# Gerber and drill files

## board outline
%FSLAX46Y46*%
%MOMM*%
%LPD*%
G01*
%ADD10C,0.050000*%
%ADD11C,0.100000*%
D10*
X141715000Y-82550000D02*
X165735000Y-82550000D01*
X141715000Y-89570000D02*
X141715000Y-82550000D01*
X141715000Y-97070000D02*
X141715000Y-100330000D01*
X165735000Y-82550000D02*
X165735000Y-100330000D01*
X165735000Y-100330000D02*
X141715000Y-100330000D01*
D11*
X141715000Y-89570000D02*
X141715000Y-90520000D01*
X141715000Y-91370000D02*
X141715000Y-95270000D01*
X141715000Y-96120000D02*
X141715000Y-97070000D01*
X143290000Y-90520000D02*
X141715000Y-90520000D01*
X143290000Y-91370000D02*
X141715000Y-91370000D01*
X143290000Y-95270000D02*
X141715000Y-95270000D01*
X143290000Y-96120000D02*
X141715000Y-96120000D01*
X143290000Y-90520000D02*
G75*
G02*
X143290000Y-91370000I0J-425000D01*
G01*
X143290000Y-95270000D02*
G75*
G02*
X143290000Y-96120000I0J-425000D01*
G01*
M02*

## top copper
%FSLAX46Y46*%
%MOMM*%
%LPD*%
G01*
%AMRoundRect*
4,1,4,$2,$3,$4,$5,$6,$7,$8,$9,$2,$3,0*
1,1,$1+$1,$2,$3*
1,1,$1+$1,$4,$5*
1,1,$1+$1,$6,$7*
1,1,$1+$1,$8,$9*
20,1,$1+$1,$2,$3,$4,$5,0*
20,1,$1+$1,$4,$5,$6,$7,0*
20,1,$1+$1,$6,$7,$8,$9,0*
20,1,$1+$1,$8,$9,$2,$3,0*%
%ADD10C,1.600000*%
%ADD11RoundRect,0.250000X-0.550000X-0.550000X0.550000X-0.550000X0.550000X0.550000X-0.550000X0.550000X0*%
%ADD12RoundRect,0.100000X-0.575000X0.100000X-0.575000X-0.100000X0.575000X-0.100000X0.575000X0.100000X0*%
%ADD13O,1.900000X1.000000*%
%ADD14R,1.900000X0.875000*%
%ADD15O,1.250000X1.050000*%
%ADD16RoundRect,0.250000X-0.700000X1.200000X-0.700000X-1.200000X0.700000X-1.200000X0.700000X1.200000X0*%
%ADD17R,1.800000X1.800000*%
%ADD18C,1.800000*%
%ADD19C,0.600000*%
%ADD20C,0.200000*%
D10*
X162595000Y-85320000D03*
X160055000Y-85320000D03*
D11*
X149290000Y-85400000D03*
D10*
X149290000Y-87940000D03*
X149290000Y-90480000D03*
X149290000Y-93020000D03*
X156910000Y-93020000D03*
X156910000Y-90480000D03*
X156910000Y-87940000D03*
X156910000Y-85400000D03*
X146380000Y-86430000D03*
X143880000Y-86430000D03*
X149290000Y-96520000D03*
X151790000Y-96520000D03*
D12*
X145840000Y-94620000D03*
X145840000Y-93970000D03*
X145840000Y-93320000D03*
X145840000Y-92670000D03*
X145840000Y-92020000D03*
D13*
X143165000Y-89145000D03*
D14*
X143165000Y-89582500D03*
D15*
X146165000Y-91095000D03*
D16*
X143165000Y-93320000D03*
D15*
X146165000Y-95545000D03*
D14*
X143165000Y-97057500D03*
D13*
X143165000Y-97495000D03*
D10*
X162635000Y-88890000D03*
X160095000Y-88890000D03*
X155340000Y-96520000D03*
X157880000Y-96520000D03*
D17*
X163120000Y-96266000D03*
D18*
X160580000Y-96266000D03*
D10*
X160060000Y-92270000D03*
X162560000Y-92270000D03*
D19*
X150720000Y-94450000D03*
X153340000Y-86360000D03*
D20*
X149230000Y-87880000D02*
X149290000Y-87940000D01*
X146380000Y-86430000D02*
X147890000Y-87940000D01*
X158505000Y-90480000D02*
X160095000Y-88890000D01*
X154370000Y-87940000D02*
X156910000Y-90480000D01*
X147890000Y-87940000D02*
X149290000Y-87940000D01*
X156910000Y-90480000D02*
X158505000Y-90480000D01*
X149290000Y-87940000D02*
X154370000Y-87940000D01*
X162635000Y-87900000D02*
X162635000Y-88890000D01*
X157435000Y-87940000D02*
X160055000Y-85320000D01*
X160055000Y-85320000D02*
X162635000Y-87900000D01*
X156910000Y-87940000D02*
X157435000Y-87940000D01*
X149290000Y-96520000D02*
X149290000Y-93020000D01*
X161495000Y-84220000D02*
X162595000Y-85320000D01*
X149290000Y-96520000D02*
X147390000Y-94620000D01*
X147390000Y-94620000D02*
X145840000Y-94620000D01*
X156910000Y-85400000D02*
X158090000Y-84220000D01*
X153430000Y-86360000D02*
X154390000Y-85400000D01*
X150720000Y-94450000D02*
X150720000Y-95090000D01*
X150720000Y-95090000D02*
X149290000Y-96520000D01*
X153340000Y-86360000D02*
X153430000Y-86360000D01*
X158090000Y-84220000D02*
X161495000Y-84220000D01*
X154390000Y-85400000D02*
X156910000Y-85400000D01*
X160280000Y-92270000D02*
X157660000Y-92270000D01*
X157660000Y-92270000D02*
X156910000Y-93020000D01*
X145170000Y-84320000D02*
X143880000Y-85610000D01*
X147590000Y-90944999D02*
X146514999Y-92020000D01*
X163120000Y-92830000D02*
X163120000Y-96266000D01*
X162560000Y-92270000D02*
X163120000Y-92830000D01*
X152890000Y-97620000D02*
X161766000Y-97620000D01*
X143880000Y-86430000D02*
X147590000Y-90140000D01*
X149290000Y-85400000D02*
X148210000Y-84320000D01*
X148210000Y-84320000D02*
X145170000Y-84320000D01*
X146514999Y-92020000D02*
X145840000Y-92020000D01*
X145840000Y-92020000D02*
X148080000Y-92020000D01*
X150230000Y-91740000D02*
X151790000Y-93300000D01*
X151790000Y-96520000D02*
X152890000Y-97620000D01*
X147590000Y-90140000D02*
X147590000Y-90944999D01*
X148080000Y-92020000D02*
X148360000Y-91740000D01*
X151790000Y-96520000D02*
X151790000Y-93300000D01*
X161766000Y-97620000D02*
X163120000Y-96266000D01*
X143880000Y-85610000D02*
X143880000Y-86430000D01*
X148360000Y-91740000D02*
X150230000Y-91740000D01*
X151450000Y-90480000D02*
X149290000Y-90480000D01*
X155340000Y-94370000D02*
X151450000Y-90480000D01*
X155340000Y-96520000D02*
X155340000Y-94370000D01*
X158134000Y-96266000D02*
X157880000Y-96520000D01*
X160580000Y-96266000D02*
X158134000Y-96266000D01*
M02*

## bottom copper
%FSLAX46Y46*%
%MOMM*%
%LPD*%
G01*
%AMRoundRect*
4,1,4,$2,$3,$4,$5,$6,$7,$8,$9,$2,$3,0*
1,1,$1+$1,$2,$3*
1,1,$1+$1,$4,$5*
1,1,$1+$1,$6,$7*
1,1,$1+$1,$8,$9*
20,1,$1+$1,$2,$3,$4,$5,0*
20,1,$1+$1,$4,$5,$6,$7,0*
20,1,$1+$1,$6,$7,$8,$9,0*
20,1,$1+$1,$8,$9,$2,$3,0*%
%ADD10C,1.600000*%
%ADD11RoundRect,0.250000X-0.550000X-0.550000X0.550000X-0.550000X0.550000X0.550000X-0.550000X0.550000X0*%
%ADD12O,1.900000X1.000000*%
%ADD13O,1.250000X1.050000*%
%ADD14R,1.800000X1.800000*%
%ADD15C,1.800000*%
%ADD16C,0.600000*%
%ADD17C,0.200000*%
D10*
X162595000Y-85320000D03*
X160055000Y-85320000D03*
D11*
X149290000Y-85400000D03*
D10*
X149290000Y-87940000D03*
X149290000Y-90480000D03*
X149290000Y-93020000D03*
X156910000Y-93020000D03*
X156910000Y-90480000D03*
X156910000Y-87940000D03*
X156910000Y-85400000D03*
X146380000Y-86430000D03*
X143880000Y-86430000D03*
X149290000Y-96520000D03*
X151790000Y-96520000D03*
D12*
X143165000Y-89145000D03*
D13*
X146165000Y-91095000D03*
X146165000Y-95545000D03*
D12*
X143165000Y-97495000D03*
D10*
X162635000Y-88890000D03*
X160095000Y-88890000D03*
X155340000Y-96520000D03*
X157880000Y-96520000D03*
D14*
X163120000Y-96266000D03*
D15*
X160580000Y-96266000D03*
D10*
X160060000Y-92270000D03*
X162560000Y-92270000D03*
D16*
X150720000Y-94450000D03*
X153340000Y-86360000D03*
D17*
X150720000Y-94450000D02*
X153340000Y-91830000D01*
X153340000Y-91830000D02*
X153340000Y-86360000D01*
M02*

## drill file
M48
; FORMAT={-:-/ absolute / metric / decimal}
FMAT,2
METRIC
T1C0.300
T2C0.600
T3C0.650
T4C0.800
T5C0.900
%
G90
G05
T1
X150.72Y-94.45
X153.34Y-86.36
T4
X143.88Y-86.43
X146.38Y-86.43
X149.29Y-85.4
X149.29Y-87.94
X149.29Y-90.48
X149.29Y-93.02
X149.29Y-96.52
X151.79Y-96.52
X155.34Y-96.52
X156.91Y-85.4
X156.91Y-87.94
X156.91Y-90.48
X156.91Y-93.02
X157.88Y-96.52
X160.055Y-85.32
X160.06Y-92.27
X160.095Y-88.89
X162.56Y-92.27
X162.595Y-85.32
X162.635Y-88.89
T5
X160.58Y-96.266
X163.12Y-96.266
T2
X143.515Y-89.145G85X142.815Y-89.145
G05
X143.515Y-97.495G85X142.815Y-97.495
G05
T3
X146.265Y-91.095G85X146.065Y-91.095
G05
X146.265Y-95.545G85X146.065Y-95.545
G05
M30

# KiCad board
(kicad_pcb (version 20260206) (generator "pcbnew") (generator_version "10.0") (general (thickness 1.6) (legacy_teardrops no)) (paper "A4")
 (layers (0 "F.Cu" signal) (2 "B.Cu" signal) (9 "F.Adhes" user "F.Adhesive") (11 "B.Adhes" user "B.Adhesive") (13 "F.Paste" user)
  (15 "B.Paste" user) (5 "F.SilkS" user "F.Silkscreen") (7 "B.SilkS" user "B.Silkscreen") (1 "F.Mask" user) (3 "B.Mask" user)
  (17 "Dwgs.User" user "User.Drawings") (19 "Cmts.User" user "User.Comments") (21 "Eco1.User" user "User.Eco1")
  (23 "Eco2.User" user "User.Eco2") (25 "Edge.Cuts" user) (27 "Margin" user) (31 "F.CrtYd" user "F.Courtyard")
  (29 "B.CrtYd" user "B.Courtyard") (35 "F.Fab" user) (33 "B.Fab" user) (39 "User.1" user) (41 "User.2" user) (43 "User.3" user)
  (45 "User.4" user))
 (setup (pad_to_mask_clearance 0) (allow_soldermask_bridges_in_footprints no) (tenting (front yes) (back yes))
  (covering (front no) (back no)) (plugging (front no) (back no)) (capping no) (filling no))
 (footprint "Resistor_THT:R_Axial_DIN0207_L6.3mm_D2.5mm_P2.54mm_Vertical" (layer "F.Cu") (at 162.595 85.32 180)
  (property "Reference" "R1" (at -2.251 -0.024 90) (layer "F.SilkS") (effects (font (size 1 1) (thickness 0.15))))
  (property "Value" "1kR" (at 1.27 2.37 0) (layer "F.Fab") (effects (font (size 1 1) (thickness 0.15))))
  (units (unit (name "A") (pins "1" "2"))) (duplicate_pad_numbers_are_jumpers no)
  (pad "1" thru_hole circle (at 0 0 180) (size 1.6 1.6) (drill 0.8) (layers "*.Cu" "*.Mask") (remove_unused_layers no) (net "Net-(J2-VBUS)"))
  (pad "2" thru_hole circle (at 2.54 0 180) (size 1.6 1.6) (drill 0.8) (layers "*.Cu" "*.Mask") (remove_unused_layers no)
   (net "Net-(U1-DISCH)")))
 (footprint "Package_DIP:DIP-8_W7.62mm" (layer "F.Cu") (at 149.29 85.4)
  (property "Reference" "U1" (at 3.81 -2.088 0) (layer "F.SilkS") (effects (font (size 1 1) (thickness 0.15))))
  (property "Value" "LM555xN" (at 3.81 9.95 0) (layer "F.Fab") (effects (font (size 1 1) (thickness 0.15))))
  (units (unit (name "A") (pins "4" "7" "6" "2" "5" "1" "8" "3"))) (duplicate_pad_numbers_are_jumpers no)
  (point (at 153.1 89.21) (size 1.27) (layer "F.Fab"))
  (pad "1" thru_hole roundrect (at 0 0) (size 1.6 1.6) (drill 0.8) (layers "*.Cu" "*.Mask") (remove_unused_layers no)
   (roundrect_rratio 0.15625) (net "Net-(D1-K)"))
  (pad "2" thru_hole circle (at 0 2.54) (size 1.6 1.6) (drill 0.8) (layers "*.Cu" "*.Mask") (remove_unused_layers no) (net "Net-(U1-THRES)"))
  (pad "3" thru_hole circle (at 0 5.08) (size 1.6 1.6) (drill 0.8) (layers "*.Cu" "*.Mask") (remove_unused_layers no) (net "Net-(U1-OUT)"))
  (pad "4" thru_hole circle (at 0 7.62) (size 1.6 1.6) (drill 0.8) (layers "*.Cu" "*.Mask") (remove_unused_layers no) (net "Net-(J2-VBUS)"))
  (pad "5" thru_hole circle (at 7.62 7.62) (size 1.6 1.6) (drill 0.8) (layers "*.Cu" "*.Mask") (remove_unused_layers no)
   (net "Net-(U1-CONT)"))
  (pad "6" thru_hole circle (at 7.62 5.08) (size 1.6 1.6) (drill 0.8) (layers "*.Cu" "*.Mask") (remove_unused_layers no)
   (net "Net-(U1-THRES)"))
  (pad "7" thru_hole circle (at 7.62 2.54) (size 1.6 1.6) (drill 0.8) (layers "*.Cu" "*.Mask") (remove_unused_layers no)
   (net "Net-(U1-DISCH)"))
  (pad "8" thru_hole circle (at 7.62 0) (size 1.6 1.6) (drill 0.8) (layers "*.Cu" "*.Mask") (remove_unused_layers no) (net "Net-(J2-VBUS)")))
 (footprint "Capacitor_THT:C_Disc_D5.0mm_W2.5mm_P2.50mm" (layer "F.Cu") (at 146.38 86.43 180)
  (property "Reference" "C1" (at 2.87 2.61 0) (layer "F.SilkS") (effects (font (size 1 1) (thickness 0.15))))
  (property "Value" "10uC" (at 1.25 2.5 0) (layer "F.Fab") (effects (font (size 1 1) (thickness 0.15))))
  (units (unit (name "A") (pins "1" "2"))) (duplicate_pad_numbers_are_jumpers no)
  (pad "1" thru_hole circle (at 0 0 180) (size 1.6 1.6) (drill 0.8) (layers "*.Cu" "*.Mask") (remove_unused_layers no)
   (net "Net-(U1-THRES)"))
  (pad "2" thru_hole circle (at 2.5 0 180) (size 1.6 1.6) (drill 0.8) (layers "*.Cu" "*.Mask") (remove_unused_layers no) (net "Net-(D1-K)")))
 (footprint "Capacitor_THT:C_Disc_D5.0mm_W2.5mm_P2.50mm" (layer "F.Cu") (at 149.29 96.52)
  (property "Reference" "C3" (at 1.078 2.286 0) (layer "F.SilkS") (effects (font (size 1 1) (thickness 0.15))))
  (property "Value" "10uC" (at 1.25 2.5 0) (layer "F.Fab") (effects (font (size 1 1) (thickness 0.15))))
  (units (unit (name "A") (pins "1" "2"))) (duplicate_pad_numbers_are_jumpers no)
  (pad "1" thru_hole circle (at 0 0) (size 1.6 1.6) (drill 0.8) (layers "*.Cu" "*.Mask") (remove_unused_layers no) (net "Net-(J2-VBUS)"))
  (pad "2" thru_hole circle (at 2.5 0) (size 1.6 1.6) (drill 0.8) (layers "*.Cu" "*.Mask") (remove_unused_layers no) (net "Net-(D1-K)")))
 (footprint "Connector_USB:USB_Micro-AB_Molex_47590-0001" (layer "F.Cu") (at 142.815 93.32 -90)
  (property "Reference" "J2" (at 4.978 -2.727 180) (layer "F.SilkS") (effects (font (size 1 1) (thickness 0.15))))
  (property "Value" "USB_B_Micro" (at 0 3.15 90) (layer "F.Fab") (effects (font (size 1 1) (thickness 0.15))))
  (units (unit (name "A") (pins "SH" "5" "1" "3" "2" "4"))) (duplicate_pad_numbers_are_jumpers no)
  (fp_line (start -3.75 1.1) (end -2.8 1.1) (stroke (width 0.1) (type solid)) (layer "Edge.Cuts"))
  (fp_line (start -1.95 1.1) (end 1.95 1.1) (stroke (width 0.1) (type solid)) (layer "Edge.Cuts"))
  (fp_line (start 2.8 1.1) (end 3.75 1.1) (stroke (width 0.1) (type solid)) (layer "Edge.Cuts"))
  (fp_line (start -2.8 -0.475) (end -2.8 1.1) (stroke (width 0.1) (type solid)) (layer "Edge.Cuts"))
  (fp_line (start -1.95 -0.475) (end -1.95 1.1) (stroke (width 0.1) (type solid)) (layer "Edge.Cuts"))
  (fp_line (start 1.95 -0.475) (end 1.95 1.1) (stroke (width 0.1) (type solid)) (layer "Edge.Cuts"))
  (fp_line (start 2.8 -0.475) (end 2.8 1.1) (stroke (width 0.1) (type solid)) (layer "Edge.Cuts"))
  (fp_arc (start -2.8 -0.475) (mid -2.375 -0.9) (end -1.95 -0.475) (stroke (width 0.1) (type solid)) (layer "Edge.Cuts"))
  (fp_arc (start 1.95 -0.475) (mid 2.375 -0.9) (end 2.8 -0.475) (stroke (width 0.1) (type solid)) (layer "Edge.Cuts"))
  (pad "" smd rect (at -3.5 -0.35 270) (size 0.3 0.85) (layers "F.Paste"))
  (pad "" smd rect (at 3.5 -0.35 270) (size 0.3 0.85) (layers "F.Paste"))
  (pad "1" smd roundrect (at 1.3 -3.025 270) (size 0.4 1.35) (layers "F.Cu" "F.Mask" "F.Paste") (roundrect_rratio 0.25)
   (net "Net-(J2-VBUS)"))
  (pad "2" smd roundrect (at 0.65 -3.025 270) (size 0.4 1.35) (layers "F.Cu" "F.Mask" "F.Paste") (roundrect_rratio 0.25)
   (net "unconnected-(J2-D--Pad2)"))
  (pad "3" smd roundrect (at 0 -3.025 270) (size 0.4 1.35) (layers "F.Cu" "F.Mask" "F.Paste") (roundrect_rratio 0.25)
   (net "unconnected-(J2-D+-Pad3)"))
  (pad "4" smd roundrect (at -0.65 -3.025 270) (size 0.4 1.35) (layers "F.Cu" "F.Mask" "F.Paste") (roundrect_rratio 0.25)
   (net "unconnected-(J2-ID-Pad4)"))
  (pad "5" smd roundrect (at -1.3 -3.025 270) (size 0.4 1.35) (layers "F.Cu" "F.Mask" "F.Paste") (roundrect_rratio 0.25) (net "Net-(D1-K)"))
  (pad "SH" thru_hole oval (at -4.175 -0.35 270) (size 1 1.9) (drill oval 0.6 1.3) (layers "*.Cu" "*.Mask") (remove_unused_layers no)
   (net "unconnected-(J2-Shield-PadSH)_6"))
  (pad "SH" smd rect (at -3.7375 -0.35 270) (size 0.875 1.9) (layers "F.Cu" "F.Mask") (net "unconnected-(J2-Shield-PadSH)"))
  (pad "SH" thru_hole oval (at -2.225 -3.35 270) (size 1.05 1.25) (drill oval 0.65 0.85) (layers "*.Cu" "*.Mask") (remove_unused_layers no)
   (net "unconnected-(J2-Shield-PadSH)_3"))
  (pad "SH" smd roundrect (at 0 -0.35 270) (size 2.9 1.9) (layers "F.Cu" "F.Mask" "F.Paste") (roundrect_rratio 0.1315789474)
   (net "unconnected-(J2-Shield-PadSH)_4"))
  (pad "SH" thru_hole oval (at 2.225 -3.35 270) (size 1.05 1.25) (drill oval 0.65 0.85) (layers "*.Cu" "*.Mask") (remove_unused_layers no)
   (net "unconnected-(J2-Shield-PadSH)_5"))
  (pad "SH" smd rect (at 3.7375 -0.35 270) (size 0.875 1.9) (layers "F.Cu" "F.Mask") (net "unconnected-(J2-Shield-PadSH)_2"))
  (pad "SH" thru_hole oval (at 4.175 -0.35 270) (size 1 1.9) (drill oval 0.6 1.3) (layers "*.Cu" "*.Mask") (remove_unused_layers no)
   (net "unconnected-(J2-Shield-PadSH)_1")))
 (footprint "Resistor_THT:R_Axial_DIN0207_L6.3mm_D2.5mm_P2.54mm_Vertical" (layer "F.Cu") (at 162.635 88.89 180)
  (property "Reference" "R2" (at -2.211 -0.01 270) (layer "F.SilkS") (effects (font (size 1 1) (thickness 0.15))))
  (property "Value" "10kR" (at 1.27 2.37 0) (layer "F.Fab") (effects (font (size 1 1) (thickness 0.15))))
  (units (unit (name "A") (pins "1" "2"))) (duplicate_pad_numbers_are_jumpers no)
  (pad "1" thru_hole circle (at 0 0 180) (size 1.6 1.6) (drill 0.8) (layers "*.Cu" "*.Mask") (remove_unused_layers no)
   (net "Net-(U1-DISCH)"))
  (pad "2" thru_hole circle (at 2.54 0 180) (size 1.6 1.6) (drill 0.8) (layers "*.Cu" "*.Mask") (remove_unused_layers no)
   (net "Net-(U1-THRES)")))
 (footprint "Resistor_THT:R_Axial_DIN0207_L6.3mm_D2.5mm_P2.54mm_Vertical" (layer "F.Cu") (at 155.34 96.52)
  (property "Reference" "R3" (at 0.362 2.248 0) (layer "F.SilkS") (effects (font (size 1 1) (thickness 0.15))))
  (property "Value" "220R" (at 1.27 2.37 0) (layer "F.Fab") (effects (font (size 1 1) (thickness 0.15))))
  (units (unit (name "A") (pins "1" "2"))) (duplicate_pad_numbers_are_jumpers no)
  (pad "1" thru_hole circle (at 0 0) (size 1.6 1.6) (drill 0.8) (layers "*.Cu" "*.Mask") (remove_unused_layers no) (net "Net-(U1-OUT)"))
  (pad "2" thru_hole circle (at 2.54 0) (size 1.6 1.6) (drill 0.8) (layers "*.Cu" "*.Mask") (remove_unused_layers no) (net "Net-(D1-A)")))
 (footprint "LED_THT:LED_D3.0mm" (layer "F.Cu") (at 163.12 96.266 180)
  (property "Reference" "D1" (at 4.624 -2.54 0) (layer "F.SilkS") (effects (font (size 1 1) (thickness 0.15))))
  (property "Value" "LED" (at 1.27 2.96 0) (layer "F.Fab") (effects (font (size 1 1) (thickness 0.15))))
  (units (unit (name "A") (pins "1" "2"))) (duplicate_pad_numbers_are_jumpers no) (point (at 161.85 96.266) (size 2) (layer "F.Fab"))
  (pad "1" thru_hole rect (at 0 0 180) (size 1.8 1.8) (drill 0.9) (layers "*.Cu" "*.Mask") (remove_unused_layers no) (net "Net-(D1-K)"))
  (pad "2" thru_hole circle (at 2.54 0 180) (size 1.8 1.8) (drill 0.9) (layers "*.Cu" "*.Mask") (remove_unused_layers no) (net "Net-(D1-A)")))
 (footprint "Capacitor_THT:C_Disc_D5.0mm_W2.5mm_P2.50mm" (layer "F.Cu") (at 160.06 92.27)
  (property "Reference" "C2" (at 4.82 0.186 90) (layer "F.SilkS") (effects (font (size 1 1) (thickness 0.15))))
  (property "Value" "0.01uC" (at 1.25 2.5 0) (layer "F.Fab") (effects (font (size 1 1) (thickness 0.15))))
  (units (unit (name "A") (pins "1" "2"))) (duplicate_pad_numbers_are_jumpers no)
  (pad "1" thru_hole circle (at 0 0) (size 1.6 1.6) (drill 0.8) (layers "*.Cu" "*.Mask") (remove_unused_layers no) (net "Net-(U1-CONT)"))
  (pad "2" thru_hole circle (at 2.5 0) (size 1.6 1.6) (drill 0.8) (layers "*.Cu" "*.Mask") (remove_unused_layers no) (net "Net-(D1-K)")))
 (gr_line (start 141.715 82.55) (end 165.735 82.55) (stroke (width 0.05) (type default)) (layer "Edge.Cuts"))
 (gr_line (start 141.715 89.57) (end 141.715 82.55) (stroke (width 0.05) (type default)) (layer "Edge.Cuts"))
 (gr_line (start 141.715 97.07) (end 141.715 100.33) (stroke (width 0.05) (type default)) (layer "Edge.Cuts"))
 (gr_line (start 165.735 82.55) (end 165.735 100.33) (stroke (width 0.05) (type default)) (layer "Edge.Cuts"))
 (gr_line (start 165.735 100.33) (end 141.715 100.33) (stroke (width 0.05) (type default)) (layer "Edge.Cuts"))
 (segment (start 149.23 87.88) (end 149.29 87.94) (width 0.2) (layer "F.Cu") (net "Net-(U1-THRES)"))
 (segment (start 146.38 86.43) (end 147.89 87.94) (width 0.2) (layer "F.Cu") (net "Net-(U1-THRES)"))
 (segment (start 158.505 90.48) (end 160.095 88.89) (width 0.2) (layer "F.Cu") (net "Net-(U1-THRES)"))
 (segment (start 154.37 87.94) (end 156.91 90.48) (width 0.2) (layer "F.Cu") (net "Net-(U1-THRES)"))
 (segment (start 147.89 87.94) (end 149.29 87.94) (width 0.2) (layer "F.Cu") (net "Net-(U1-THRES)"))
 (segment (start 156.91 90.48) (end 158.505 90.48) (width 0.2) (layer "F.Cu") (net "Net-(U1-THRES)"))
 (segment (start 149.29 87.94) (end 154.37 87.94) (width 0.2) (layer "F.Cu") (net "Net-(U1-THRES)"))
 (segment (start 162.635 87.9) (end 162.635 88.89) (width 0.2) (layer "F.Cu") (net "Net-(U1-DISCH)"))
 (segment (start 157.435 87.94) (end 160.055 85.32) (width 0.2) (layer "F.Cu") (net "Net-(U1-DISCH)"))
 (segment (start 160.055 85.32) (end 162.635 87.9) (width 0.2) (layer "F.Cu") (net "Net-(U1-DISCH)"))
 (segment (start 156.91 87.94) (end 157.435 87.94) (width 0.2) (layer "F.Cu") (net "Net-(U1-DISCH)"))
 (segment (start 149.29 96.52) (end 149.29 93.02) (width 0.2) (layer "F.Cu") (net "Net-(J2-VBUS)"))
 (segment (start 161.495 84.22) (end 162.595 85.32) (width 0.2) (layer "F.Cu") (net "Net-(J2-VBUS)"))
 (segment (start 149.29 96.52) (end 147.39 94.62) (width 0.2) (layer "F.Cu") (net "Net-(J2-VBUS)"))
 (segment (start 147.39 94.62) (end 145.84 94.62) (width 0.2) (layer "F.Cu") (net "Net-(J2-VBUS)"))
 (segment (start 156.91 85.4) (end 158.09 84.22) (width 0.2) (layer "F.Cu") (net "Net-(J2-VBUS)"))
 (segment (start 153.43 86.36) (end 154.39 85.4) (width 0.2) (layer "F.Cu") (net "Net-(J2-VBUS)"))
 (segment (start 150.72 94.45) (end 150.72 95.09) (width 0.2) (layer "F.Cu") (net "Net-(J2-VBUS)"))
 (segment (start 150.72 95.09) (end 149.29 96.52) (width 0.2) (layer "F.Cu") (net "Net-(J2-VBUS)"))
 (segment (start 153.34 86.36) (end 153.43 86.36) (width 0.2) (layer "F.Cu") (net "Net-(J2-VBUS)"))
 (segment (start 158.09 84.22) (end 161.495 84.22) (width 0.2) (layer "F.Cu") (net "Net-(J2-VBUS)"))
 (segment (start 154.39 85.4) (end 156.91 85.4) (width 0.2) (layer "F.Cu") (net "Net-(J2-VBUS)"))
 (via (at 150.72 94.45) (size 0.6) (drill 0.3) (layers "F.Cu" "B.Cu") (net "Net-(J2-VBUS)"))
 (via (at 153.34 86.36) (size 0.6) (drill 0.3) (layers "F.Cu" "B.Cu") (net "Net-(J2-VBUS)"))
 (segment (start 150.72 94.45) (end 153.34 91.83) (width 0.2) (layer "B.Cu") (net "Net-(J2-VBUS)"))
 (segment (start 153.34 91.83) (end 153.34 86.36) (width 0.2) (layer "B.Cu") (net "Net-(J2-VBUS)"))
 (segment (start 160.28 92.27) (end 157.66 92.27) (width 0.2) (layer "F.Cu") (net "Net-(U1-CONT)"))
 (segment (start 157.66 92.27) (end 156.91 93.02) (width 0.2) (layer "F.Cu") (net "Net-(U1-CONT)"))
 (segment (start 145.17 84.32) (end 143.88 85.61) (width 0.2) (layer "F.Cu") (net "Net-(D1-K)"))
 (segment (start 147.59 90.944999) (end 146.514999 92.02) (width 0.2) (layer "F.Cu") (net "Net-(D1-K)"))
 (segment (start 163.12 92.83) (end 163.12 96.266) (width 0.2) (layer "F.Cu") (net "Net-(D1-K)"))
 (segment (start 162.56 92.27) (end 163.12 92.83) (width 0.2) (layer "F.Cu") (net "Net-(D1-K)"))
 (segment (start 152.89 97.62) (end 161.766 97.62) (width 0.2) (layer "F.Cu") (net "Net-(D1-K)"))
 (segment (start 143.88 86.43) (end 147.59 90.14) (width 0.2) (layer "F.Cu") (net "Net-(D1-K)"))
 (segment (start 149.29 85.4) (end 148.21 84.32) (width 0.2) (layer "F.Cu") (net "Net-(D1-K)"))
 (segment (start 148.21 84.32) (end 145.17 84.32) (width 0.2) (layer "F.Cu") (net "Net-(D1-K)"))
 (segment (start 146.514999 92.02) (end 145.84 92.02) (width 0.2) (layer "F.Cu") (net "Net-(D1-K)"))
 (segment (start 145.84 92.02) (end 148.08 92.02) (width 0.2) (layer "F.Cu") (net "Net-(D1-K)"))
 (segment (start 150.23 91.74) (end 151.79 93.3) (width 0.2) (layer "F.Cu") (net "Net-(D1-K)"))
 (segment (start 151.79 96.52) (end 152.89 97.62) (width 0.2) (layer "F.Cu") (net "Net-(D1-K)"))
 (segment (start 147.59 90.14) (end 147.59 90.944999) (width 0.2) (layer "F.Cu") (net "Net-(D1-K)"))
 (segment (start 148.08 92.02) (end 148.36 91.74) (width 0.2) (layer "F.Cu") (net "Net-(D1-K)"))
 (segment (start 151.79 96.52) (end 151.79 93.3) (width 0.2) (layer "F.Cu") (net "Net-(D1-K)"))
 (segment (start 161.766 97.62) (end 163.12 96.266) (width 0.2) (layer "F.Cu") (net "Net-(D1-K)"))
 (segment (start 143.88 85.61) (end 143.88 86.43) (width 0.2) (layer "F.Cu") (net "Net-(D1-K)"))
 (segment (start 148.36 91.74) (end 150.23 91.74) (width 0.2) (layer "F.Cu") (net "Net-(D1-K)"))
 (segment (start 151.45 90.48) (end 149.29 90.48) (width 0.2) (layer "F.Cu") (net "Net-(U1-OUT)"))
 (segment (start 155.34 94.37) (end 151.45 90.48) (width 0.2) (layer "F.Cu") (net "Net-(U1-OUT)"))
 (segment (start 155.34 96.52) (end 155.34 94.37) (width 0.2) (layer "F.Cu") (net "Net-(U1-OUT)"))
 (segment (start 158.134 96.266) (end 157.88 96.52) (width 0.2) (layer "F.Cu") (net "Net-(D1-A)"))
 (segment (start 160.58 96.266) (end 158.134 96.266) (width 0.2) (layer "F.Cu") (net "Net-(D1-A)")))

